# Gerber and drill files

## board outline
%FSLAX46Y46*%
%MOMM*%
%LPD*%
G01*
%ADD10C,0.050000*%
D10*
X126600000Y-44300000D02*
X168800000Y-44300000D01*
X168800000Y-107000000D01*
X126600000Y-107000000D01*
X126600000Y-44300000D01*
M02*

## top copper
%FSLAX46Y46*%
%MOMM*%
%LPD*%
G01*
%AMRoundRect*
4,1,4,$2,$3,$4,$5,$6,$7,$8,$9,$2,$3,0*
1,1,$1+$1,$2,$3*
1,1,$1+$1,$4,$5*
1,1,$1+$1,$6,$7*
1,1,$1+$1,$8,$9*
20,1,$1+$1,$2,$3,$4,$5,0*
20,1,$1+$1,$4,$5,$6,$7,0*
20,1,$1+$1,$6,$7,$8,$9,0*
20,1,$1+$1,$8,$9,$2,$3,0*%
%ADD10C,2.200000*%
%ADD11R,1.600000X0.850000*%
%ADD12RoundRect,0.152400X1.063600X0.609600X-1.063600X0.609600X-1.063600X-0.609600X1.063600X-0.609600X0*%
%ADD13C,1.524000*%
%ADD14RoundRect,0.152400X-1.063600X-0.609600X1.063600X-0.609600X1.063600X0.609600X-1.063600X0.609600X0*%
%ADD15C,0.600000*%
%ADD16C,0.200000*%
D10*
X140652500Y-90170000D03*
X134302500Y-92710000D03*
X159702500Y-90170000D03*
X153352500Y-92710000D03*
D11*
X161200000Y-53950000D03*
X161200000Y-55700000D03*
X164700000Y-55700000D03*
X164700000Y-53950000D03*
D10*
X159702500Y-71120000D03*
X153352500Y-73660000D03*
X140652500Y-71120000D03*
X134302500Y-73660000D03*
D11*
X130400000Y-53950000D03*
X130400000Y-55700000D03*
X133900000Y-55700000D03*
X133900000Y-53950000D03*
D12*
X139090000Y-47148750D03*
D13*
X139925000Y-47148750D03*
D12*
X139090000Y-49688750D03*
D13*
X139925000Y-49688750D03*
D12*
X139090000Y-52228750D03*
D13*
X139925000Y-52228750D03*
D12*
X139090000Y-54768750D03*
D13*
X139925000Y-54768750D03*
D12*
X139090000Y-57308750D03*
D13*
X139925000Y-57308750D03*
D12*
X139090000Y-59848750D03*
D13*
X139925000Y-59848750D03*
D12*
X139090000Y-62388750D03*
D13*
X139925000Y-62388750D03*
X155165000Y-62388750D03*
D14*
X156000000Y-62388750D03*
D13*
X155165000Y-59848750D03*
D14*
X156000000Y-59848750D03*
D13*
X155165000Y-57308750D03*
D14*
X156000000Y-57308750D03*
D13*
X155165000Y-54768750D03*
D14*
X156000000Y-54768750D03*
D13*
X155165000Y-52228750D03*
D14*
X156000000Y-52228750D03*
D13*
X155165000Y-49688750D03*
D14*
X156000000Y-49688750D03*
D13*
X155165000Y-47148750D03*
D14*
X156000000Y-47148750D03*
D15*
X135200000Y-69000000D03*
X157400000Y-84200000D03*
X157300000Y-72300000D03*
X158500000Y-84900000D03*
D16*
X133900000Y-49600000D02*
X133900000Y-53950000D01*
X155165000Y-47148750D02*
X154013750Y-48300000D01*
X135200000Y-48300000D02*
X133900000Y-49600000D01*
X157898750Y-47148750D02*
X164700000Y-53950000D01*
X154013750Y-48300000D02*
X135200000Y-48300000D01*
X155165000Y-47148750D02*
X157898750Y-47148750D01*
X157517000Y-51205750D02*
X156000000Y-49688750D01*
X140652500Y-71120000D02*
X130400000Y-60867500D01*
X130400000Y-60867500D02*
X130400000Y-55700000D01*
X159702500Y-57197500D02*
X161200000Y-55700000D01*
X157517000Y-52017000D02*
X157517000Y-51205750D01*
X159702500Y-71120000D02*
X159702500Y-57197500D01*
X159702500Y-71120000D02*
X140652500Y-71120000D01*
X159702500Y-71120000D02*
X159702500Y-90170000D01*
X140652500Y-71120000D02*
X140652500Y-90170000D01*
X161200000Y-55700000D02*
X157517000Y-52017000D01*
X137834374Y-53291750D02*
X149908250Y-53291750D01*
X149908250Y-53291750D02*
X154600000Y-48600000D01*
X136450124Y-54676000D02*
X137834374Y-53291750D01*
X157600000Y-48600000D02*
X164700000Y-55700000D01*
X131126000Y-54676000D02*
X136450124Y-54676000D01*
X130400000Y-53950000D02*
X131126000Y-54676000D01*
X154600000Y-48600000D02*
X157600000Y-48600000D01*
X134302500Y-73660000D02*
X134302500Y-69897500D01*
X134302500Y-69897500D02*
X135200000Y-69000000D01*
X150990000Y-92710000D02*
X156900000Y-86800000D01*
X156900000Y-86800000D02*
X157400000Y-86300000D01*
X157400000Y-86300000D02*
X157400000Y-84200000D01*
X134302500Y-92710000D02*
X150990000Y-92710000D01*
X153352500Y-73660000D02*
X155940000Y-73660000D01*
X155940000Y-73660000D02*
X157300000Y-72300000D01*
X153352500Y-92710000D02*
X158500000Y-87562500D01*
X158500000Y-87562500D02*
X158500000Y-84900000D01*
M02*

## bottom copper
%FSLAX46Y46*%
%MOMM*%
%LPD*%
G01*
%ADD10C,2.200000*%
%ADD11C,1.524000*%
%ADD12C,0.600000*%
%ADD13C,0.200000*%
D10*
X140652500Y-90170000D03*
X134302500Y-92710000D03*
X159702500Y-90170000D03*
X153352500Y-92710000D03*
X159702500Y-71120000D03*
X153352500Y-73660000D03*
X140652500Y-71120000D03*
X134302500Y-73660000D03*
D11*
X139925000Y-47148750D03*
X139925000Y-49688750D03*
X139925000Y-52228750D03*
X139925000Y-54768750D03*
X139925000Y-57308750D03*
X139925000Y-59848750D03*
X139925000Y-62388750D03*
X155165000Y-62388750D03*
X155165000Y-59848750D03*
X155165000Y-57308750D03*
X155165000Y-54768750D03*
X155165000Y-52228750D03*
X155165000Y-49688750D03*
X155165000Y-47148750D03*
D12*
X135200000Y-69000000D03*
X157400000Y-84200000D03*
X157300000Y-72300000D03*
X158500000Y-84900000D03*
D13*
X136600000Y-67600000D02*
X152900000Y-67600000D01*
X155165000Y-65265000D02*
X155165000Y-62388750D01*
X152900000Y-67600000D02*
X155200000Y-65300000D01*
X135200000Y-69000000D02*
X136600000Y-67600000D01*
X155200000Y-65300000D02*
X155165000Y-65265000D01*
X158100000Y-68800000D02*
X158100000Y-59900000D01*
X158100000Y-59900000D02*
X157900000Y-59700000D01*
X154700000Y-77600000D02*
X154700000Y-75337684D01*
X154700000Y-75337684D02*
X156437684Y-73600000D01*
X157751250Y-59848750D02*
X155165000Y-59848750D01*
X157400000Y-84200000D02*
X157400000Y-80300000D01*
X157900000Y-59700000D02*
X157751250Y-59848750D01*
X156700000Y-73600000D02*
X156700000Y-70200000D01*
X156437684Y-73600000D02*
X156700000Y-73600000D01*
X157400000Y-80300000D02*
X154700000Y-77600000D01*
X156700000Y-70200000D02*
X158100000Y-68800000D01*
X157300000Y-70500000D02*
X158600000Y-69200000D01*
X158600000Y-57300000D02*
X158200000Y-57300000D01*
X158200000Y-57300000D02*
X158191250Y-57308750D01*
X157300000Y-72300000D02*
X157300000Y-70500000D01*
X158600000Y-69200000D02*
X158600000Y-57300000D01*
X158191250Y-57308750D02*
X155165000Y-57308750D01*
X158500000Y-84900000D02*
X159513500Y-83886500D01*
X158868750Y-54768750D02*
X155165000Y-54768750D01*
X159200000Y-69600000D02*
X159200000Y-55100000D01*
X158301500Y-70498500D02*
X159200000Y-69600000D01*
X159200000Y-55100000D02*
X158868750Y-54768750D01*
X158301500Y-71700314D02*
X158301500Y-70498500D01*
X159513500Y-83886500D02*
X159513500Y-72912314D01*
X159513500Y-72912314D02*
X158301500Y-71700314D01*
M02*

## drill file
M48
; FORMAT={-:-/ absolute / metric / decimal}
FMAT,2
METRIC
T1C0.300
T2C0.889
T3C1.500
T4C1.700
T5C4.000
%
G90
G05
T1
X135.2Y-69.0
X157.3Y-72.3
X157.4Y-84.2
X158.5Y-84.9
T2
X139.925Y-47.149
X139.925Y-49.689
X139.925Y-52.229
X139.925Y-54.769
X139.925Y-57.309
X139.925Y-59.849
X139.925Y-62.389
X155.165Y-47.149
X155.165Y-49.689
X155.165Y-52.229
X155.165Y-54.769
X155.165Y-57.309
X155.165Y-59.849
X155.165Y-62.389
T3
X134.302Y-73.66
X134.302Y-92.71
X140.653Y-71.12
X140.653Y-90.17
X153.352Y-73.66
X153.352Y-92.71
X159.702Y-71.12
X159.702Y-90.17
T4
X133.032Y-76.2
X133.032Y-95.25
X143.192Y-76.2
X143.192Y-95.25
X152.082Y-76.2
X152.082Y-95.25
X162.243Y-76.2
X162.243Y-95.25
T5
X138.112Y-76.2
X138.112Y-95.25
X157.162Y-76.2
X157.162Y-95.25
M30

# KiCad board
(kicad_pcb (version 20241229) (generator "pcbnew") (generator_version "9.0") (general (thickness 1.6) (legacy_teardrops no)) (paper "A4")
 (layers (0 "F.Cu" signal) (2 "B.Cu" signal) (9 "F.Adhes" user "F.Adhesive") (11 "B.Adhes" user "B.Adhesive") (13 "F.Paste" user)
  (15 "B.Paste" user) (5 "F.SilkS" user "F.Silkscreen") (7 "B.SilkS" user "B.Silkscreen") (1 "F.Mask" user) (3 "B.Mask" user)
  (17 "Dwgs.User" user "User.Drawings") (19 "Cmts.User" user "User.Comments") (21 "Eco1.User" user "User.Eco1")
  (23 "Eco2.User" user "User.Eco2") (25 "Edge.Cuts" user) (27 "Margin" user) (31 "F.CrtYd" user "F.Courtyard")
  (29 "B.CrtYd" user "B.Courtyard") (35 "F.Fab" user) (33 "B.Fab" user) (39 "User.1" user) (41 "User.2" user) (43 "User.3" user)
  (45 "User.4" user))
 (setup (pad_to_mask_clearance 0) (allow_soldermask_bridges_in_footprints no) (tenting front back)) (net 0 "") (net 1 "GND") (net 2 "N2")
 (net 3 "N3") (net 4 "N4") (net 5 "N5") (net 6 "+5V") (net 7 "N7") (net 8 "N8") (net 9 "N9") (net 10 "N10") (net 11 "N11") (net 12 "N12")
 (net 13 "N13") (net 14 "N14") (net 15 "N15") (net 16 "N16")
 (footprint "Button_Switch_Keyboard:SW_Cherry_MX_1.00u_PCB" (layer "F.Cu") (at 140.6525 90.17)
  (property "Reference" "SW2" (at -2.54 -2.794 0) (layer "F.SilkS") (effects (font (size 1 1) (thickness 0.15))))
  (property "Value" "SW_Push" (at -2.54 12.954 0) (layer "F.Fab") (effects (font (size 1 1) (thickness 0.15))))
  (pad "" np_thru_hole circle (at -7.62 5.08) (size 1.7 1.7) (drill 1.7) (layers "*.Cu" "*.Mask"))
  (pad "" np_thru_hole circle (at -2.54 5.08) (size 4 4) (drill 4) (layers "*.Cu" "*.Mask"))
  (pad "" np_thru_hole circle (at 2.54 5.08) (size 1.7 1.7) (drill 1.7) (layers "*.Cu" "*.Mask"))
  (pad "1" thru_hole circle (at 0 0) (size 2.2 2.2) (drill 1.5) (layers "*.Cu" "*.Mask") (remove_unused_layers no) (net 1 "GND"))
  (pad "2" thru_hole circle (at -6.35 2.54) (size 2.2 2.2) (drill 1.5) (layers "*.Cu" "*.Mask") (remove_unused_layers no) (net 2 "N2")))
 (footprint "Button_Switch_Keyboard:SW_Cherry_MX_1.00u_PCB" (layer "F.Cu") (at 159.7025 90.17)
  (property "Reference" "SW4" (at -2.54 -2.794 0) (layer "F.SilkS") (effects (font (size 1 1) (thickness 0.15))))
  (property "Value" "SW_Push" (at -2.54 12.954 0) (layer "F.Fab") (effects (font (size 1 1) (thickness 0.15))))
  (pad "" np_thru_hole circle (at -7.62 5.08) (size 1.7 1.7) (drill 1.7) (layers "*.Cu" "*.Mask"))
  (pad "" np_thru_hole circle (at -2.54 5.08) (size 4 4) (drill 4) (layers "*.Cu" "*.Mask"))
  (pad "" np_thru_hole circle (at 2.54 5.08) (size 1.7 1.7) (drill 1.7) (layers "*.Cu" "*.Mask"))
  (pad "1" thru_hole circle (at 0 0) (size 2.2 2.2) (drill 1.5) (layers "*.Cu" "*.Mask") (remove_unused_layers no) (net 1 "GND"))
  (pad "2" thru_hole circle (at -6.35 2.54) (size 2.2 2.2) (drill 1.5) (layers "*.Cu" "*.Mask") (remove_unused_layers no) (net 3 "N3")))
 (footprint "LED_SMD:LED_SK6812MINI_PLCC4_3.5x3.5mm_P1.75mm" (layer "F.Cu") (at 162.95 54.825)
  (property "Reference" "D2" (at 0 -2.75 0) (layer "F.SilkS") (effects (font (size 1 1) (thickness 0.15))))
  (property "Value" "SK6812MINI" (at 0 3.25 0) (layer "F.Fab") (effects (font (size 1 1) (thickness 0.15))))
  (pad "1" smd rect (at -1.75 -0.875) (size 1.6 0.85) (layers "F.Cu" "F.Mask" "F.Paste") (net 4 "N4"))
  (pad "2" smd rect (at -1.75 0.875) (size 1.6 0.85) (layers "F.Cu" "F.Mask" "F.Paste") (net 1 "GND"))
  (pad "3" smd rect (at 1.75 0.875) (size 1.6 0.85) (layers "F.Cu" "F.Mask" "F.Paste") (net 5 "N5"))
  (pad "4" smd rect (at 1.75 -0.875) (size 1.6 0.85) (layers "F.Cu" "F.Mask" "F.Paste") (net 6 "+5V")))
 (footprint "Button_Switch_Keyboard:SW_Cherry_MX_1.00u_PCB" (layer "F.Cu") (at 159.7025 71.12)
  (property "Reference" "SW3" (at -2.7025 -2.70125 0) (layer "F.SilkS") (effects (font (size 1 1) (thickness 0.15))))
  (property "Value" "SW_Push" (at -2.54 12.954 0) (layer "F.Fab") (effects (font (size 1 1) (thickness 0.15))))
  (pad "" np_thru_hole circle (at -7.62 5.08) (size 1.7 1.7) (drill 1.7) (layers "*.Cu" "*.Mask"))
  (pad "" np_thru_hole circle (at -2.54 5.08) (size 4 4) (drill 4) (layers "*.Cu" "*.Mask"))
  (pad "" np_thru_hole circle (at 2.54 5.08) (size 1.7 1.7) (drill 1.7) (layers "*.Cu" "*.Mask"))
  (pad "1" thru_hole circle (at 0 0) (size 2.2 2.2) (drill 1.5) (layers "*.Cu" "*.Mask") (remove_unused_layers no) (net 1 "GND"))
  (pad "2" thru_hole circle (at -6.35 2.54) (size 2.2 2.2) (drill 1.5) (layers "*.Cu" "*.Mask") (remove_unused_layers no) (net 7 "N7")))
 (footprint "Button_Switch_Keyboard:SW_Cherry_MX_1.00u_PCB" (layer "F.Cu") (at 140.6525 71.12)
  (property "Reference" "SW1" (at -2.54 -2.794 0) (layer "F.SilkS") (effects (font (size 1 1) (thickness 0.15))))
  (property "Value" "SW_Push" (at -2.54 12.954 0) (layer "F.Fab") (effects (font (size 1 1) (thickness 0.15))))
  (pad "" np_thru_hole circle (at -7.62 5.08) (size 1.7 1.7) (drill 1.7) (layers "*.Cu" "*.Mask"))
  (pad "" np_thru_hole circle (at -2.54 5.08) (size 4 4) (drill 4) (layers "*.Cu" "*.Mask"))
  (pad "" np_thru_hole circle (at 2.54 5.08) (size 1.7 1.7) (drill 1.7) (layers "*.Cu" "*.Mask"))
  (pad "1" thru_hole circle (at 0 0) (size 2.2 2.2) (drill 1.5) (layers "*.Cu" "*.Mask") (remove_unused_layers no) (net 1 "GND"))
  (pad "2" thru_hole circle (at -6.35 2.54) (size 2.2 2.2) (drill 1.5) (layers "*.Cu" "*.Mask") (remove_unused_layers no) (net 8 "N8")))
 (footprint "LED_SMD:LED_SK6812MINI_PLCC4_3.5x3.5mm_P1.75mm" (layer "F.Cu") (at 132.15 54.825)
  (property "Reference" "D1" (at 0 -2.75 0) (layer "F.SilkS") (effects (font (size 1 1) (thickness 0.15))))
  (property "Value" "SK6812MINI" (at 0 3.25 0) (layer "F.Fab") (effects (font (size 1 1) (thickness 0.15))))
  (pad "1" smd rect (at -1.75 -0.875) (size 1.6 0.85) (layers "F.Cu" "F.Mask" "F.Paste") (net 5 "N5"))
  (pad "2" smd rect (at -1.75 0.875) (size 1.6 0.85) (layers "F.Cu" "F.Mask" "F.Paste") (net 1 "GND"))
  (pad "3" smd rect (at 1.75 0.875) (size 1.6 0.85) (layers "F.Cu" "F.Mask" "F.Paste") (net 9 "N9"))
  (pad "4" smd rect (at 1.75 -0.875) (size 1.6 0.85) (layers "F.Cu" "F.Mask" "F.Paste") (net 6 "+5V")))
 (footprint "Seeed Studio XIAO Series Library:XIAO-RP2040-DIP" (layer "F.Cu") (at 147.545 54.76875)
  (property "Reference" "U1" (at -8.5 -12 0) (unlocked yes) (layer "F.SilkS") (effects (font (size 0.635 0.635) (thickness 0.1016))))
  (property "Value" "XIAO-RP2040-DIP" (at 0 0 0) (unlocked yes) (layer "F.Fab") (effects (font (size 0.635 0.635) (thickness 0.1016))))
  (pad "1" smd roundrect (at -8.455 -7.62 180) (size 2.432 1.524) (layers "F.Cu" "F.Mask") (roundrect_rratio 0.1) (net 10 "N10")
   (thermal_bridge_angle 45))
  (pad "1" thru_hole circle (at -7.62 -7.62 180) (size 1.524 1.524) (drill 0.889) (layers "*.Cu" "*.Mask") (remove_unused_layers no)
   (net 10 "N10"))
  (pad "2" smd roundrect (at -8.455 -5.08 180) (size 2.432 1.524) (layers "F.Cu" "F.Mask") (roundrect_rratio 0.1) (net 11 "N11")
   (thermal_bridge_angle 45))
  (pad "2" thru_hole circle (at -7.62 -5.08 180) (size 1.524 1.524) (drill 0.889) (layers "*.Cu" "*.Mask") (remove_unused_layers no)
   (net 11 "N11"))
  (pad "3" smd roundrect (at -8.455 -2.54 180) (size 2.432 1.524) (layers "F.Cu" "F.Mask") (roundrect_rratio 0.1) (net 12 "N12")
   (thermal_bridge_angle 45))
  (pad "3" thru_hole circle (at -7.62 -2.54 180) (size 1.524 1.524) (drill 0.889) (layers "*.Cu" "*.Mask") (remove_unused_layers no)
   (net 12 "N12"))
  (pad "4" smd roundrect (at -8.455 0 180) (size 2.432 1.524) (layers "F.Cu" "F.Mask") (roundrect_rratio 0.1) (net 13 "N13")
   (thermal_bridge_angle 45))
  (pad "4" thru_hole circle (at -7.62 0 180) (size 1.524 1.524) (drill 0.889) (layers "*.Cu" "*.Mask") (remove_unused_layers no)
   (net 13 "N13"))
  (pad "5" smd roundrect (at -8.455 2.54 180) (size 2.432 1.524) (layers "F.Cu" "F.Mask") (roundrect_rratio 0.1) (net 9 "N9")
   (thermal_bridge_angle 45))
  (pad "5" thru_hole circle (at -7.62 2.54 180) (size 1.524 1.524) (drill 0.889) (layers "*.Cu" "*.Mask") (remove_unused_layers no)
   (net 9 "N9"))
  (pad "6" smd roundrect (at -8.455 5.08 180) (size 2.432 1.524) (layers "F.Cu" "F.Mask") (roundrect_rratio 0.1) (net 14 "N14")
   (thermal_bridge_angle 45))
  (pad "6" thru_hole circle (at -7.62 5.08 180) (size 1.524 1.524) (drill 0.889) (layers "*.Cu" "*.Mask") (remove_unused_layers no)
   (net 14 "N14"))
  (pad "7" smd roundrect (at -8.455 7.62 180) (size 2.432 1.524) (layers "F.Cu" "F.Mask") (roundrect_rratio 0.1) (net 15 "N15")
   (thermal_bridge_angle 45))
  (pad "7" thru_hole circle (at -7.62 7.62 180) (size 1.524 1.524) (drill 0.889) (layers "*.Cu" "*.Mask") (remove_unused_layers no)
   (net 15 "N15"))
  (pad "8" thru_hole circle (at 7.62 7.62) (size 1.524 1.524) (drill 0.889) (layers "*.Cu" "*.Mask") (remove_unused_layers no) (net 8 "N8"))
  (pad "8" smd roundrect (at 8.455 7.62) (size 2.432 1.524) (layers "F.Cu" "F.Mask") (roundrect_rratio 0.1) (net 8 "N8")
   (thermal_bridge_angle 45))
  (pad "9" thru_hole circle (at 7.62 5.08) (size 1.524 1.524) (drill 0.889) (layers "*.Cu" "*.Mask") (remove_unused_layers no) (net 2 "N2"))
  (pad "9" smd roundrect (at 8.455 5.08) (size 2.432 1.524) (layers "F.Cu" "F.Mask") (roundrect_rratio 0.1) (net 2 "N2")
   (thermal_bridge_angle 45))
  (pad "10" thru_hole circle (at 7.62 2.54) (size 1.524 1.524) (drill 0.889) (layers "*.Cu" "*.Mask") (remove_unused_layers no) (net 7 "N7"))
  (pad "10" smd roundrect (at 8.455 2.54) (size 2.432 1.524) (layers "F.Cu" "F.Mask") (roundrect_rratio 0.1) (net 7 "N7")
   (thermal_bridge_angle 45))
  (pad "11" thru_hole circle (at 7.62 0) (size 1.524 1.524) (drill 0.889) (layers "*.Cu" "*.Mask") (remove_unused_layers no) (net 3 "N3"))
  (pad "11" smd roundrect (at 8.455 0) (size 2.432 1.524) (layers "F.Cu" "F.Mask") (roundrect_rratio 0.1) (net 3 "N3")
   (thermal_bridge_angle 45))
  (pad "12" thru_hole circle (at 7.62 -2.54) (size 1.524 1.524) (drill 0.889) (layers "*.Cu" "*.Mask") (remove_unused_layers no)
   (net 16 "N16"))
  (pad "12" smd roundrect (at 8.455 -2.54) (size 2.432 1.524) (layers "F.Cu" "F.Mask") (roundrect_rratio 0.1) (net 16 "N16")
   (thermal_bridge_angle 45))
  (pad "13" thru_hole circle (at 7.62 -5.08) (size 1.524 1.524) (drill 0.889) (layers "*.Cu" "*.Mask") (remove_unused_layers no)
   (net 1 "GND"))
  (pad "13" smd roundrect (at 8.455 -5.08) (size 2.432 1.524) (layers "F.Cu" "F.Mask") (roundrect_rratio 0.1) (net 1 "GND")
   (thermal_bridge_angle 45))
  (pad "14" thru_hole circle (at 7.62 -7.62) (size 1.524 1.524) (drill 0.889) (layers "*.Cu" "*.Mask") (remove_unused_layers no)
   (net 6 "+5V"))
  (pad "14" smd roundrect (at 8.455 -7.62) (size 2.432 1.524) (layers "F.Cu" "F.Mask") (roundrect_rratio 0.1) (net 6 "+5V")
   (thermal_bridge_angle 45)))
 (gr_rect (start 126.6 44.3) (end 168.8 107) (stroke (width 0.05) (type default)) (fill no) (layer "Edge.Cuts"))
 (segment (start 133.9 49.6) (end 133.9 53.95) (width 0.2) (layer "F.Cu") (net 6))
 (segment (start 155.165 47.14875) (end 154.01375 48.3) (width 0.2) (layer "F.Cu") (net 6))
 (segment (start 135.2 48.3) (end 133.9 49.6) (width 0.2) (layer "F.Cu") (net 6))
 (segment (start 157.89875 47.14875) (end 164.7 53.95) (width 0.2) (layer "F.Cu") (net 6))
 (segment (start 154.01375 48.3) (end 135.2 48.3) (width 0.2) (layer "F.Cu") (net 6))
 (segment (start 155.165 47.14875) (end 157.89875 47.14875) (width 0.2) (layer "F.Cu") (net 6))
 (segment (start 157.517 51.20575) (end 156 49.68875) (width 0.2) (layer "F.Cu") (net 1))
 (segment (start 140.6525 71.12) (end 130.4 60.8675) (width 0.2) (layer "F.Cu") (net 1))
 (segment (start 130.4 60.8675) (end 130.4 55.7) (width 0.2) (layer "F.Cu") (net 1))
 (segment (start 159.7025 57.1975) (end 161.2 55.7) (width 0.2) (layer "F.Cu") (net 1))
 (segment (start 157.517 52.017) (end 157.517 51.20575) (width 0.2) (layer "F.Cu") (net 1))
 (segment (start 159.7025 71.12) (end 159.7025 57.1975) (width 0.2) (layer "F.Cu") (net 1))
 (segment (start 159.7025 71.12) (end 140.6525 71.12) (width 0.2) (layer "F.Cu") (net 1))
 (segment (start 159.7025 71.12) (end 159.7025 90.17) (width 0.2) (layer "F.Cu") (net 1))
 (segment (start 140.6525 71.12) (end 140.6525 90.17) (width 0.2) (layer "F.Cu") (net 1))
 (segment (start 161.2 55.7) (end 157.517 52.017) (width 0.2) (layer "F.Cu") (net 1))
 (segment (start 137.834374 53.29175) (end 149.90825 53.29175) (width 0.2) (layer "F.Cu") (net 5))
 (segment (start 149.90825 53.29175) (end 154.6 48.6) (width 0.2) (layer "F.Cu") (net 5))
 (segment (start 136.450124 54.676) (end 137.834374 53.29175) (width 0.2) (layer "F.Cu") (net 5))
 (segment (start 157.6 48.6) (end 164.7 55.7) (width 0.2) (layer "F.Cu") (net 5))
 (segment (start 131.126 54.676) (end 136.450124 54.676) (width 0.2) (layer "F.Cu") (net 5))
 (segment (start 130.4 53.95) (end 131.126 54.676) (width 0.2) (layer "F.Cu") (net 5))
 (segment (start 154.6 48.6) (end 157.6 48.6) (width 0.2) (layer "F.Cu") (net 5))
 (segment (start 134.3025 73.66) (end 134.3025 69.8975) (width 0.2) (layer "F.Cu") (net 8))
 (segment (start 134.3025 69.8975) (end 135.2 69) (width 0.2) (layer "F.Cu") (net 8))
 (via (at 135.2 69) (size 0.6) (drill 0.3) (layers "F.Cu" "B.Cu") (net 8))
 (segment (start 136.6 67.6) (end 152.9 67.6) (width 0.2) (layer "B.Cu") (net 8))
 (segment (start 155.165 65.265) (end 155.165 62.38875) (width 0.2) (layer "B.Cu") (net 8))
 (segment (start 152.9 67.6) (end 155.2 65.3) (width 0.2) (layer "B.Cu") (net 8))
 (segment (start 135.2 69) (end 136.6 67.6) (width 0.2) (layer "B.Cu") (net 8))
 (segment (start 155.2 65.3) (end 155.165 65.265) (width 0.2) (layer "B.Cu") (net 8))
 (segment (start 150.99 92.71) (end 156.9 86.8) (width 0.2) (layer "F.Cu") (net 2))
 (segment (start 156.9 86.8) (end 157.4 86.3) (width 0.2) (layer "F.Cu") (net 2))
 (segment (start 157.4 86.3) (end 157.4 84.2) (width 0.2) (layer "F.Cu") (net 2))
 (segment (start 134.3025 92.71) (end 150.99 92.71) (width 0.2) (layer "F.Cu") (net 2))
 (via (at 157.4 84.2) (size 0.6) (drill 0.3) (layers "F.Cu" "B.Cu") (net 2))
 (segment (start 158.1 68.8) (end 158.1 59.9) (width 0.2) (layer "B.Cu") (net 2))
 (segment (start 158.1 59.9) (end 157.9 59.7) (width 0.2) (layer "B.Cu") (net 2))
 (segment (start 154.7 77.6) (end 154.7 75.337684) (width 0.2) (layer "B.Cu") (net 2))
 (segment (start 154.7 75.337684) (end 156.437684 73.6) (width 0.2) (layer "B.Cu") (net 2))
 (segment (start 157.75125 59.84875) (end 155.165 59.84875) (width 0.2) (layer "B.Cu") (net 2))
 (segment (start 157.4 84.2) (end 157.4 80.3) (width 0.2) (layer "B.Cu") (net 2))
 (segment (start 157.9 59.7) (end 157.75125 59.84875) (width 0.2) (layer "B.Cu") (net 2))
 (segment (start 156.7 73.6) (end 156.7 70.2) (width 0.2) (layer "B.Cu") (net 2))
 (segment (start 156.437684 73.6) (end 156.7 73.6) (width 0.2) (layer "B.Cu") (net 2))
 (segment (start 157.4 80.3) (end 154.7 77.6) (width 0.2) (layer "B.Cu") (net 2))
 (segment (start 156.7 70.2) (end 158.1 68.8) (width 0.2) (layer "B.Cu") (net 2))
 (segment (start 153.3525 73.66) (end 155.94 73.66) (width 0.2) (layer "F.Cu") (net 7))
 (segment (start 155.94 73.66) (end 157.3 72.3) (width 0.2) (layer "F.Cu") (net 7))
 (via (at 157.3 72.3) (size 0.6) (drill 0.3) (layers "F.Cu" "B.Cu") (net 7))
 (segment (start 157.3 70.5) (end 158.6 69.2) (width 0.2) (layer "B.Cu") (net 7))
 (segment (start 158.6 57.3) (end 158.2 57.3) (width 0.2) (layer "B.Cu") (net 7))
 (segment (start 158.2 57.3) (end 158.19125 57.30875) (width 0.2) (layer "B.Cu") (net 7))
 (segment (start 157.3 72.3) (end 157.3 70.5) (width 0.2) (layer "B.Cu") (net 7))
 (segment (start 158.6 69.2) (end 158.6 57.3) (width 0.2) (layer "B.Cu") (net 7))
 (segment (start 158.19125 57.30875) (end 155.165 57.30875) (width 0.2) (layer "B.Cu") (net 7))
 (segment (start 153.3525 92.71) (end 158.5 87.5625) (width 0.2) (layer "F.Cu") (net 3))
 (segment (start 158.5 87.5625) (end 158.5 84.9) (width 0.2) (layer "F.Cu") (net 3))
 (via (at 158.5 84.9) (size 0.6) (drill 0.3) (layers "F.Cu" "B.Cu") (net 3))
 (segment (start 158.5 84.9) (end 159.5135 83.8865) (width 0.2) (layer "B.Cu") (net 3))
 (segment (start 158.86875 54.76875) (end 155.165 54.76875) (width 0.2) (layer "B.Cu") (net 3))
 (segment (start 159.2 69.6) (end 159.2 55.1) (width 0.2) (layer "B.Cu") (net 3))
 (segment (start 158.3015 70.4985) (end 159.2 69.6) (width 0.2) (layer "B.Cu") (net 3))
 (segment (start 159.2 55.1) (end 158.86875 54.76875) (width 0.2) (layer "B.Cu") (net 3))
 (segment (start 158.3015 71.700314) (end 158.3015 70.4985) (width 0.2) (layer "B.Cu") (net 3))
 (segment (start 159.5135 83.8865) (end 159.5135 72.912314) (width 0.2) (layer "B.Cu") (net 3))
 (segment (start 159.5135 72.912314) (end 158.3015 71.700314) (width 0.2) (layer "B.Cu") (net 3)))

